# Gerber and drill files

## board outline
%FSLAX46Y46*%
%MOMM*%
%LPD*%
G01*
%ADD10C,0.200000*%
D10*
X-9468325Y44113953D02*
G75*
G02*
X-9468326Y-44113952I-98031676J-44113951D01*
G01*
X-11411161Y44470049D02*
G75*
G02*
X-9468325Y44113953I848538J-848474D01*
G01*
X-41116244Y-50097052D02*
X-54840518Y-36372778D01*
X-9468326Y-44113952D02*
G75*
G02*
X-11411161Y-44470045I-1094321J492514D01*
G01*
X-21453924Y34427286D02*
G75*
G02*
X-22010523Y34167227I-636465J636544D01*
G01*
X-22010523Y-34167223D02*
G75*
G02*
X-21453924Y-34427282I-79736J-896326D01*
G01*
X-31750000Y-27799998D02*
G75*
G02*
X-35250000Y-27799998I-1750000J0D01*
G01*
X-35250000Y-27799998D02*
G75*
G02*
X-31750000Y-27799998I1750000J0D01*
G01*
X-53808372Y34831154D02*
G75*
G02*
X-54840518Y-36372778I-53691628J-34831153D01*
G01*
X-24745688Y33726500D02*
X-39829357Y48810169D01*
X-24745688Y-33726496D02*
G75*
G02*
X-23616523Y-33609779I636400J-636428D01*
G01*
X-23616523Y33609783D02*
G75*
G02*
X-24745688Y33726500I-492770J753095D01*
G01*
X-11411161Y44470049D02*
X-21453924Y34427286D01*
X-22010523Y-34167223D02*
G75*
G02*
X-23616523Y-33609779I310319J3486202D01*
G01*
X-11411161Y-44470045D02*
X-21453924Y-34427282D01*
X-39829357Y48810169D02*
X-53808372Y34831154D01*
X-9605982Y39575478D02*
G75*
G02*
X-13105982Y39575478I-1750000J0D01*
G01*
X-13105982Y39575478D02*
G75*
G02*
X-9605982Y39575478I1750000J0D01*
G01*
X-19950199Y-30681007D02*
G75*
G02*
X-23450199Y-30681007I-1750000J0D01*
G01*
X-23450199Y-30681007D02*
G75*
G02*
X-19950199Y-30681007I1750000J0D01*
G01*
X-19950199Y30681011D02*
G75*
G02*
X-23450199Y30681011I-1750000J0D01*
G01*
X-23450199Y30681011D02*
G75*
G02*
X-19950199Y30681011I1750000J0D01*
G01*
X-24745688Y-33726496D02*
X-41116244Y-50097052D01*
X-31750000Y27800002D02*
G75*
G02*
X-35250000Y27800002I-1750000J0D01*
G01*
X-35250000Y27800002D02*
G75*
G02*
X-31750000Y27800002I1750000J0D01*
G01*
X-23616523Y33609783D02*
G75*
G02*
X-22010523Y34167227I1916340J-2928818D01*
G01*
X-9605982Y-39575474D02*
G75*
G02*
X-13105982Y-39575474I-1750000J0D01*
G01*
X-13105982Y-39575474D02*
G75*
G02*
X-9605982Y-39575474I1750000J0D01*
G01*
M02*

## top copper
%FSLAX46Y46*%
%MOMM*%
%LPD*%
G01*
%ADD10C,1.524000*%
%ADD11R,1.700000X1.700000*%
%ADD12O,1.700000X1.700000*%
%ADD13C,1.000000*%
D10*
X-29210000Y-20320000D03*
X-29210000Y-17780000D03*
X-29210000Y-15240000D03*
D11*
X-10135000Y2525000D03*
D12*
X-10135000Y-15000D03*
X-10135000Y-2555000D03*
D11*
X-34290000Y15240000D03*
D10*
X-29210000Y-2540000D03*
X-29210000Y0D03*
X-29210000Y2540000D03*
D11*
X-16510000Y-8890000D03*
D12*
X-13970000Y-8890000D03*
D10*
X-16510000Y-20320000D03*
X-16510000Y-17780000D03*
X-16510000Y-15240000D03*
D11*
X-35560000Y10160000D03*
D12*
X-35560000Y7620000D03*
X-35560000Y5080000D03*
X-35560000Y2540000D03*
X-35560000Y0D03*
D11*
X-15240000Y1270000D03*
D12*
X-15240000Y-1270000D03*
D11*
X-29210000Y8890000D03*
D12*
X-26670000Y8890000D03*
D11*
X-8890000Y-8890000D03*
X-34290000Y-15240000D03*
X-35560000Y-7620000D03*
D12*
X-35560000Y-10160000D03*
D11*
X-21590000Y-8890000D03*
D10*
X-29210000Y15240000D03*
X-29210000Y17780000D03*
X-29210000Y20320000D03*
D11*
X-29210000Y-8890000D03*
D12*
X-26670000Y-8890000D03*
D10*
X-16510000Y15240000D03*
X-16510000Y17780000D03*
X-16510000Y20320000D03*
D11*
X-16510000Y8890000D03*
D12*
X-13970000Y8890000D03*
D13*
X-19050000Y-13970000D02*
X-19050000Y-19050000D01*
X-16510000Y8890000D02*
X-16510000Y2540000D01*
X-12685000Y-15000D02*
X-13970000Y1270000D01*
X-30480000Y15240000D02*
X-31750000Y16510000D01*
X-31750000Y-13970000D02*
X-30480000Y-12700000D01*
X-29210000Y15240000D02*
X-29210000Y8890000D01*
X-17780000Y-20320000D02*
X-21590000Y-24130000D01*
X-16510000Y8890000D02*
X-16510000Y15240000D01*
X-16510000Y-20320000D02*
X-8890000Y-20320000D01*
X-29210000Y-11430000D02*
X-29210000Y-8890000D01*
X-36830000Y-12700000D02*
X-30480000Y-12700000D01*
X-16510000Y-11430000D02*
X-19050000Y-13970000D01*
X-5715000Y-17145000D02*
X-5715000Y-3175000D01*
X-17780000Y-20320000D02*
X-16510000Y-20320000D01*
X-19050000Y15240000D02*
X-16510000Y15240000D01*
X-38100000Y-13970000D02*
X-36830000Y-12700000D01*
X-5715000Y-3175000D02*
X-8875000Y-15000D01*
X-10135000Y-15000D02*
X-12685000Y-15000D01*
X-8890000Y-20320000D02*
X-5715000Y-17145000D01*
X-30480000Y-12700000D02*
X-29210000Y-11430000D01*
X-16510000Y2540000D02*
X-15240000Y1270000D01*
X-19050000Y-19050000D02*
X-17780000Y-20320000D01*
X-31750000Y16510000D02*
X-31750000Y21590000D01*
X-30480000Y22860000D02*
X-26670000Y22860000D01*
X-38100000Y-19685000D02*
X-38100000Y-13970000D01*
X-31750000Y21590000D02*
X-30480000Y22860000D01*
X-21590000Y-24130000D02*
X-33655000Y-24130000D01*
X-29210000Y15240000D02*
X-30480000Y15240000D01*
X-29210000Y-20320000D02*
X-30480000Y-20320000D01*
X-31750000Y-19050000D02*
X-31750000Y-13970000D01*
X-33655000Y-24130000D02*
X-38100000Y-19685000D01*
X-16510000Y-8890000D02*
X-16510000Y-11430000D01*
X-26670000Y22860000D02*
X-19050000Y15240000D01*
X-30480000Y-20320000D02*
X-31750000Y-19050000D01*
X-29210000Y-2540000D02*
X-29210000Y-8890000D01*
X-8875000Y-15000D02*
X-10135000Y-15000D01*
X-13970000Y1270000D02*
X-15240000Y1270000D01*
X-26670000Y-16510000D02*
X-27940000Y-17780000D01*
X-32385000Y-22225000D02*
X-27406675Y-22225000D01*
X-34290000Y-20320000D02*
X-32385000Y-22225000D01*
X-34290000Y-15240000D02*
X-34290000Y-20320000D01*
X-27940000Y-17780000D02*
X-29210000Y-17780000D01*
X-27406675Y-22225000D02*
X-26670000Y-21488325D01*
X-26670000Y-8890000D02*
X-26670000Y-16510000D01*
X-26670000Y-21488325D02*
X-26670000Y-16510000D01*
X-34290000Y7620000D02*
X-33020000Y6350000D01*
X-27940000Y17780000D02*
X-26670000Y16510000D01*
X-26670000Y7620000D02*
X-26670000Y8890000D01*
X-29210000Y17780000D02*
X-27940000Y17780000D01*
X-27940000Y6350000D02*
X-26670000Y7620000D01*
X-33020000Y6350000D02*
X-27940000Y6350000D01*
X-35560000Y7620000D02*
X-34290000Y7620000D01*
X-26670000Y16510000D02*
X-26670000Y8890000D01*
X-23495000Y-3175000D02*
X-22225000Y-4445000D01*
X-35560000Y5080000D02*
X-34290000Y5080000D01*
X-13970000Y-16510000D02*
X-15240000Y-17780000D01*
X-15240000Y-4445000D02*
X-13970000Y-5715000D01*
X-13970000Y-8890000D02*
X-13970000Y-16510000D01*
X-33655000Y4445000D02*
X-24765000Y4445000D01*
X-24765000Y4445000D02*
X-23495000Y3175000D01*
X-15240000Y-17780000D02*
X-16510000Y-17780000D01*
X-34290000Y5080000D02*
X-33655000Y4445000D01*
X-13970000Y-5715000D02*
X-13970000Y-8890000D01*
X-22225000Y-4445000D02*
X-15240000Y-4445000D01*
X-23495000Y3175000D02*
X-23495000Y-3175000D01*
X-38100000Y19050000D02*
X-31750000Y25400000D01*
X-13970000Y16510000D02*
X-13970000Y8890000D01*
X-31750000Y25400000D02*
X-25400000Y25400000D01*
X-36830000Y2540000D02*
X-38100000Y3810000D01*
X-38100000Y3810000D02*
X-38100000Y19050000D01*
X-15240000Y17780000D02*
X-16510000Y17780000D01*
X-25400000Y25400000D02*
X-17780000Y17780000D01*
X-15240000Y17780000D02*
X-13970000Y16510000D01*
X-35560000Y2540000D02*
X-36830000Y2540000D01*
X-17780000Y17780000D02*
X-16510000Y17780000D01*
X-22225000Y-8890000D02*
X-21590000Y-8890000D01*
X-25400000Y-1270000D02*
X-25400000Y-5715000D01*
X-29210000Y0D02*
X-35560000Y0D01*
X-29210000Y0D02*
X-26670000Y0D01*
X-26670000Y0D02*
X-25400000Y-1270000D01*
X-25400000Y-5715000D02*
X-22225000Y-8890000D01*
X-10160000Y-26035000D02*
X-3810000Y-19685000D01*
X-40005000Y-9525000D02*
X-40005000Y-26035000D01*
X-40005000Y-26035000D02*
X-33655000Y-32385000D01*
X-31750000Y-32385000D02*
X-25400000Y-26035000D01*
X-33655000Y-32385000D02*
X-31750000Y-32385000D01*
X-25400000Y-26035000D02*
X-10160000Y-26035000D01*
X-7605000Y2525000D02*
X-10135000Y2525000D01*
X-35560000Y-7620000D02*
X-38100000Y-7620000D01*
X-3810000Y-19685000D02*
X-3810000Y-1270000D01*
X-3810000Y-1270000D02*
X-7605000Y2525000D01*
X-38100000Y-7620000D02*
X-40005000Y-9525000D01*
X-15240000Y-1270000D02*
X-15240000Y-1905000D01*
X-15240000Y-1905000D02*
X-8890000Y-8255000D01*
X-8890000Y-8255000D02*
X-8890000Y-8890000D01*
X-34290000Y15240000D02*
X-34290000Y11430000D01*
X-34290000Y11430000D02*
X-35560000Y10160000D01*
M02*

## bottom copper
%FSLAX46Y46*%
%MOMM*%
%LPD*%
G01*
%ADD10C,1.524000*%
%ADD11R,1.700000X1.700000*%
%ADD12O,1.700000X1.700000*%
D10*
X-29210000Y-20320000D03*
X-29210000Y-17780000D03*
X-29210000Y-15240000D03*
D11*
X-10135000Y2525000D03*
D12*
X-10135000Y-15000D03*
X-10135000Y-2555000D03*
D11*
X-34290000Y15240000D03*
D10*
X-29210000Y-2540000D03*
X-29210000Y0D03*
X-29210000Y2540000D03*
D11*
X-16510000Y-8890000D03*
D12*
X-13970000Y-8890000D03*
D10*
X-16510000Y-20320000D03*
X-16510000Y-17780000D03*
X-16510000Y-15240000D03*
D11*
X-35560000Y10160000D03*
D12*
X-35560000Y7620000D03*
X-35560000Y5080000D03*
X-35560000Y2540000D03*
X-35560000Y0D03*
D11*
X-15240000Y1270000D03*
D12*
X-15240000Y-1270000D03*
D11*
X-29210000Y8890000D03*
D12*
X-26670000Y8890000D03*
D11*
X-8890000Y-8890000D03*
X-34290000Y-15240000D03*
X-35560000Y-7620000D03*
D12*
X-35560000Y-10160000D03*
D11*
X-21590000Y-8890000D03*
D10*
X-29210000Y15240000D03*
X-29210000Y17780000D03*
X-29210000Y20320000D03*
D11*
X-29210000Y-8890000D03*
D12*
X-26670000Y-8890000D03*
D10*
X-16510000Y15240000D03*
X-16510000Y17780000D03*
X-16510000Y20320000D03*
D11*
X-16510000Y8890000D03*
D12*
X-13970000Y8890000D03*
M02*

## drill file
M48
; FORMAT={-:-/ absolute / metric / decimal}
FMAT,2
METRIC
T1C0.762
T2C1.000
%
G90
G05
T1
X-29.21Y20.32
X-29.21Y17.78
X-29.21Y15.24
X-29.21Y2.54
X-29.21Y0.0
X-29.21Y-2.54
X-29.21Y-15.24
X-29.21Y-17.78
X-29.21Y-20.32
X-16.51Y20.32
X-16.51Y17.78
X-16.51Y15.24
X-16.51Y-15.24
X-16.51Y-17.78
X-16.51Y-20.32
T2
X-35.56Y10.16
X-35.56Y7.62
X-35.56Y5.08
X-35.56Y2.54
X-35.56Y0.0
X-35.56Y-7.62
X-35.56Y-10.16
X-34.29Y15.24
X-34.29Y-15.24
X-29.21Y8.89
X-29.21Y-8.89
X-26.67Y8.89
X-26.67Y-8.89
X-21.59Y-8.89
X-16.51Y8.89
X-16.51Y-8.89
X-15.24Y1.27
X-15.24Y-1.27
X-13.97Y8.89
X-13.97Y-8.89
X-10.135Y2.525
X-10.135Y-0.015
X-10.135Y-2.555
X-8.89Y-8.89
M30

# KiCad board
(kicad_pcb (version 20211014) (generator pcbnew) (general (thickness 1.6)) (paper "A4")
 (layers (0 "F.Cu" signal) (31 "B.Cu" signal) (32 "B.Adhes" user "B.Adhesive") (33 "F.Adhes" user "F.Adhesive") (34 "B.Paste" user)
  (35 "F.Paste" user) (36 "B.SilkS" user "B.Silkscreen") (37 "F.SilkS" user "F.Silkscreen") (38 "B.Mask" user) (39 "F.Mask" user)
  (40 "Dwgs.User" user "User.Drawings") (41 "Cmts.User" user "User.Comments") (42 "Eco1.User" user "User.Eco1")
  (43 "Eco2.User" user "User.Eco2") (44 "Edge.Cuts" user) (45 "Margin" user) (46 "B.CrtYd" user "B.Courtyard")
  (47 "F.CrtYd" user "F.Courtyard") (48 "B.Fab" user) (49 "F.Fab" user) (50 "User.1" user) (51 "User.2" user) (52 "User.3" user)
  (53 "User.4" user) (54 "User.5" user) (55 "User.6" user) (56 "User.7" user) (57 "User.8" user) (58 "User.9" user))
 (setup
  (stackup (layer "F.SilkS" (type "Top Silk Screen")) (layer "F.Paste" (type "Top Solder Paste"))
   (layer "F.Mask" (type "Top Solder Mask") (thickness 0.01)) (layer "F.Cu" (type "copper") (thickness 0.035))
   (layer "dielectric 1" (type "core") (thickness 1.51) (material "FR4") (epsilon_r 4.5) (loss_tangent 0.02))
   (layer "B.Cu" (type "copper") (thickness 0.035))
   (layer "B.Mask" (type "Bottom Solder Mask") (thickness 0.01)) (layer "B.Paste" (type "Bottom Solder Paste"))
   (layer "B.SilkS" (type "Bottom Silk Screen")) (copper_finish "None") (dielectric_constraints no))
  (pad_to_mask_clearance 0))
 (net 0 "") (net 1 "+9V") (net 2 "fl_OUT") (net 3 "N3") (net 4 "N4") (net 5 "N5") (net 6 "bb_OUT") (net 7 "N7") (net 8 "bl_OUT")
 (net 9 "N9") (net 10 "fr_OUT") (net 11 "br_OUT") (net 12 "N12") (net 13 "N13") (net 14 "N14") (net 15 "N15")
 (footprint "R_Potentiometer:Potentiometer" (layer "F.Cu") (at -31.75 17.78 90)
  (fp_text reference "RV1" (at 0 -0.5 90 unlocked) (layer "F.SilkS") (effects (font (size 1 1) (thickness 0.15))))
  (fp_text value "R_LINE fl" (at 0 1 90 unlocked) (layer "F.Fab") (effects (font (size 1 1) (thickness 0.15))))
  (pad "1" thru_hole circle (at -2.54 2.54 90) (size 1.524 1.524) (drill 0.762) (layers *.Cu *.Mask) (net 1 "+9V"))
  (pad "2" thru_hole circle (at 0 2.54 90) (size 1.524 1.524) (drill 0.762) (layers *.Cu *.Mask) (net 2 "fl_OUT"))
  (pad "3" thru_hole circle (at 2.54 2.54 90) (size 1.524 1.524) (drill 0.762) (layers *.Cu *.Mask) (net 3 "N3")))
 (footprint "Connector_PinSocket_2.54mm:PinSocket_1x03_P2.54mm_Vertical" (layer "F.Cu") (at -10.135 -2.525)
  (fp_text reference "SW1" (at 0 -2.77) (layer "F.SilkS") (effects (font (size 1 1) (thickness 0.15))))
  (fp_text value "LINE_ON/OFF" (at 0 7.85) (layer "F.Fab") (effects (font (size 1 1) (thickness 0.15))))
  (pad "1" thru_hole rect (at 0 0) (size 1.7 1.7) (drill 1) (layers *.Cu *.Mask) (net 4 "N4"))
  (pad "2" thru_hole oval (at 0 2.54) (size 1.7 1.7) (drill 1) (layers *.Cu *.Mask) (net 1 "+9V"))
  (pad "3" thru_hole oval (at 0 5.08) (size 1.7 1.7) (drill 1) (layers *.Cu *.Mask)))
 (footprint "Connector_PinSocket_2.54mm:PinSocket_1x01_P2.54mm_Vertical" (layer "F.Cu") (at -34.29 -15.24)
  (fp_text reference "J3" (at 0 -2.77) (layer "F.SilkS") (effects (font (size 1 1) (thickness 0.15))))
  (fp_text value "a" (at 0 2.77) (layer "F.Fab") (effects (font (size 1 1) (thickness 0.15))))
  (pad "1" thru_hole rect (at 0 0) (size 1.7 1.7) (drill 1) (layers *.Cu *.Mask) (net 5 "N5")))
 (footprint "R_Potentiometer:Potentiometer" (layer "F.Cu") (at -31.75 0 90)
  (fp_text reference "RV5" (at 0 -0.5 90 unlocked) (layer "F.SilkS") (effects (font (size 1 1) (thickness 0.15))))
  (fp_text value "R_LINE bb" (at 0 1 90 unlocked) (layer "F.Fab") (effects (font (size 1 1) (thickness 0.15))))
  (pad "1" thru_hole circle (at -2.54 2.54 90) (size 1.524 1.524) (drill 0.762) (layers *.Cu *.Mask) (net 1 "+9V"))
  (pad "2" thru_hole circle (at 0 2.54 90) (size 1.524 1.524) (drill 0.762) (layers *.Cu *.Mask) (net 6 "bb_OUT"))
  (pad "3" thru_hole circle (at 2.54 2.54 90) (size 1.524 1.524) (drill 0.762) (layers *.Cu *.Mask) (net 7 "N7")))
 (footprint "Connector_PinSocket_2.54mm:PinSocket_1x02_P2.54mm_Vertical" (layer "F.Cu") (at -16.51 8.89 90)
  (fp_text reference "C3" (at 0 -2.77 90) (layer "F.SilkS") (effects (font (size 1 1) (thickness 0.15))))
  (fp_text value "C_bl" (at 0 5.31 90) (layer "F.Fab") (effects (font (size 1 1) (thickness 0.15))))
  (pad "1" thru_hole rect (at 0 0 90) (size 1.7 1.7) (drill 1) (layers *.Cu *.Mask) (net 1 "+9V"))
  (pad "2" thru_hole oval (at 0 2.54 90) (size 1.7 1.7) (drill 1) (layers *.Cu *.Mask) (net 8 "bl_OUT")))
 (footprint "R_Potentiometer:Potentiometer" (layer "F.Cu") (at -19.05 17.78 90)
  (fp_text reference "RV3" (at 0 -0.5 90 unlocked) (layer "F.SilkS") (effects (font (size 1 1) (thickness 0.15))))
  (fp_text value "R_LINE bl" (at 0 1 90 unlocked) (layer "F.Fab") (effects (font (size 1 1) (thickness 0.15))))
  (pad "1" thru_hole circle (at -2.54 2.54 90) (size 1.524 1.524) (drill 0.762) (layers *.Cu *.Mask) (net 1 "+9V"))
  (pad "2" thru_hole circle (at 0 2.54 90) (size 1.524 1.524) (drill 0.762) (layers *.Cu *.Mask) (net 8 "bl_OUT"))
  (pad "3" thru_hole circle (at 2.54 2.54 90) (size 1.524 1.524) (drill 0.762) (layers *.Cu *.Mask) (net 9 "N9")))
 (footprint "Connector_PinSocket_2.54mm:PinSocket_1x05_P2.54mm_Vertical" (layer "F.Cu") (at -35.56 -10.16)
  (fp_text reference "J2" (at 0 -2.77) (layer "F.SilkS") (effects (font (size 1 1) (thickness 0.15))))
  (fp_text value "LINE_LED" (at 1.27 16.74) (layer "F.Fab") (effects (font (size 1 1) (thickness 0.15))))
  (pad "1" thru_hole rect (at 0 0) (size 1.7 1.7) (drill 1) (layers *.Cu *.Mask) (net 5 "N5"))
  (pad "2" thru_hole oval (at 0 2.54) (size 1.7 1.7) (drill 1) (layers *.Cu *.Mask) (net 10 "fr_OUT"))
  (pad "3" thru_hole oval (at 0 5.08) (size 1.7 1.7) (drill 1) (layers *.Cu *.Mask) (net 8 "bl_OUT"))
  (pad "4" thru_hole oval (at 0 7.62) (size 1.7 1.7) (drill 1) (layers *.Cu *.Mask) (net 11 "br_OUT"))
  (pad "5" thru_hole oval (at 0 10.16) (size 1.7 1.7) (drill 1) (layers *.Cu *.Mask) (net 6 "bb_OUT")))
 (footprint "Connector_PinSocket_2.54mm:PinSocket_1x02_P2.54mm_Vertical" (layer "F.Cu") (at -15.24 -1.27)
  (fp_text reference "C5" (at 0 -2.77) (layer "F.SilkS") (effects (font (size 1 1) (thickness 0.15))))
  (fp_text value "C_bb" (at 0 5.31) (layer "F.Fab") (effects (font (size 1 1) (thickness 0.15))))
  (pad "1" thru_hole rect (at 0 0) (size 1.7 1.7) (drill 1) (layers *.Cu *.Mask) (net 1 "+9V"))
  (pad "2" thru_hole oval (at 0 2.54) (size 1.7 1.7) (drill 1) (layers *.Cu *.Mask) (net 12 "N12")))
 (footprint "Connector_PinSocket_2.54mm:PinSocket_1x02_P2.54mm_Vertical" (layer "F.Cu") (at -29.21 -8.89 90)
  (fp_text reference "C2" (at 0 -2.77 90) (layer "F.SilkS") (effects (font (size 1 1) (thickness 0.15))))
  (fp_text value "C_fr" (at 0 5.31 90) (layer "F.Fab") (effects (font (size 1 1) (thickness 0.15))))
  (pad "1" thru_hole rect (at 0 0 90) (size 1.7 1.7) (drill 1) (layers *.Cu *.Mask) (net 1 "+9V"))
  (pad "2" thru_hole oval (at 0 2.54 90) (size 1.7 1.7) (drill 1) (layers *.Cu *.Mask) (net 10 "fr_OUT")))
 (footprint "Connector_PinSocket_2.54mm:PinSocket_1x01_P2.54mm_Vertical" (layer "F.Cu") (at -8.89 8.89)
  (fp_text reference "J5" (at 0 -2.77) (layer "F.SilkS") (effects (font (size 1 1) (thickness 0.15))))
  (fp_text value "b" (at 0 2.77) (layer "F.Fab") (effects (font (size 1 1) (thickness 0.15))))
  (pad "1" thru_hole rect (at 0 0) (size 1.7 1.7) (drill 1) (layers *.Cu *.Mask) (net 12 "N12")))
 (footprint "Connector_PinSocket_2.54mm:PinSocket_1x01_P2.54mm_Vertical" (layer "F.Cu") (at -34.29 15.24)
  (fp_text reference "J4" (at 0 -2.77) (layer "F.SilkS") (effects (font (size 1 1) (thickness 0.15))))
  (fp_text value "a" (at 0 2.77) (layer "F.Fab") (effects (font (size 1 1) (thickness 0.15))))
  (pad "1" thru_hole rect (at 0 0) (size 1.7 1.7) (drill 1) (layers *.Cu *.Mask) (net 2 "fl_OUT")))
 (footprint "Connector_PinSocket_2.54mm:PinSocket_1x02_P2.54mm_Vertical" (layer "F.Cu") (at -35.56 7.62)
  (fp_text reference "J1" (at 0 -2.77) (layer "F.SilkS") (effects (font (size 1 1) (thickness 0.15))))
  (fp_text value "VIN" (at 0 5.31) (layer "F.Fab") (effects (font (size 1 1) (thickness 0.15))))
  (pad "1" thru_hole rect (at 0 0) (size 1.7 1.7) (drill 1) (layers *.Cu *.Mask) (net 4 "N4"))
  (pad "2" thru_hole oval (at 0 2.54) (size 1.7 1.7) (drill 1) (layers *.Cu *.Mask) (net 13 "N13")))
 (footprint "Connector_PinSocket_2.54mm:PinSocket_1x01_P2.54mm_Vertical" (layer "F.Cu") (at -21.59 8.89)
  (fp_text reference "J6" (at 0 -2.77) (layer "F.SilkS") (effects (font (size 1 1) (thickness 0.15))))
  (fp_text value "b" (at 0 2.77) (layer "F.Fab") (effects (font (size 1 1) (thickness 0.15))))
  (pad "1" thru_hole rect (at 0 0) (size 1.7 1.7) (drill 1) (layers *.Cu *.Mask) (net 6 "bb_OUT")))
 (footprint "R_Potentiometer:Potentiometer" (layer "F.Cu") (at -31.75 -17.78 90)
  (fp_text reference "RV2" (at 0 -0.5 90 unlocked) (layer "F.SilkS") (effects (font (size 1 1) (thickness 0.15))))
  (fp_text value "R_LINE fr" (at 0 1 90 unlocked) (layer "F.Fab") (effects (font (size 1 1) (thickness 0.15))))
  (pad "1" thru_hole circle (at -2.54 2.54 90) (size 1.524 1.524) (drill 0.762) (layers *.Cu *.Mask) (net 1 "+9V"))
  (pad "2" thru_hole circle (at 0 2.54 90) (size 1.524 1.524) (drill 0.762) (layers *.Cu *.Mask) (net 10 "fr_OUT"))
  (pad "3" thru_hole circle (at 2.54 2.54 90) (size 1.524 1.524) (drill 0.762) (layers *.Cu *.Mask) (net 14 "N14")))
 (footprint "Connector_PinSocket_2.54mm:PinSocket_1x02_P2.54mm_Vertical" (layer "F.Cu") (at -29.21 8.89 90)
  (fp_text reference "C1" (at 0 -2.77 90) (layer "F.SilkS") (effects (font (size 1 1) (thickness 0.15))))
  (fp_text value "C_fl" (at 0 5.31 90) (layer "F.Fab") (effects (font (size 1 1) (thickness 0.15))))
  (pad "1" thru_hole rect (at 0 0 90) (size 1.7 1.7) (drill 1) (layers *.Cu *.Mask) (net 1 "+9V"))
  (pad "2" thru_hole oval (at 0 2.54 90) (size 1.7 1.7) (drill 1) (layers *.Cu *.Mask) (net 2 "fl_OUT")))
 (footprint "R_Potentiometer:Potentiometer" (layer "F.Cu") (at -19.05 -17.78 90)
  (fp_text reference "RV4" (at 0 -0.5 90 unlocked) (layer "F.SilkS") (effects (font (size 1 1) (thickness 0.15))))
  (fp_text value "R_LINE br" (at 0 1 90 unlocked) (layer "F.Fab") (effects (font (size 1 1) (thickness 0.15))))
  (pad "1" thru_hole circle (at -2.54 2.54 90) (size 1.524 1.524) (drill 0.762) (layers *.Cu *.Mask) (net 1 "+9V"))
  (pad "2" thru_hole circle (at 0 2.54 90) (size 1.524 1.524) (drill 0.762) (layers *.Cu *.Mask) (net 11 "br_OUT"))
  (pad "3" thru_hole circle (at 2.54 2.54 90) (size 1.524 1.524) (drill 0.762) (layers *.Cu *.Mask) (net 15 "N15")))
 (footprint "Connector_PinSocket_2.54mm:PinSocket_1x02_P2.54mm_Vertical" (layer "F.Cu") (at -16.51 -8.89 90)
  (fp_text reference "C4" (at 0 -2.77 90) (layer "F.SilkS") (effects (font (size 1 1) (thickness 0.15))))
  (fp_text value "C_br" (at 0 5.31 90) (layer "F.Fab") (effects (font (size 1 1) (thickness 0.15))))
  (pad "1" thru_hole rect (at 0 0 90) (size 1.7 1.7) (drill 1) (layers *.Cu *.Mask) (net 1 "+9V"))
  (pad "2" thru_hole oval (at 0 2.54 90) (size 1.7 1.7) (drill 1) (layers *.Cu *.Mask) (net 11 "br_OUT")))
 (gr_arc (start -9.468325 -44.113953) (mid 0 0) (end -9.468326 44.113952) (layer "Edge.Cuts") (width 0.2))
 (gr_arc (start -11.411161 -44.470049) (mid -10.346273 -44.801879) (end -9.468325 -44.113953) (layer "Edge.Cuts") (width 0.2))
 (gr_line (start -41.116244 50.097052) (end -54.840518 36.372778) (layer "Edge.Cuts") (width 0.2))
 (gr_arc (start -9.468326 44.113952) (mid -10.346285 44.801818) (end -11.411161 44.470045) (layer "Edge.Cuts") (width 0.2))
 (gr_arc (start -21.453924 -34.427286) (mid -21.709349 -34.248303) (end -22.010523 -34.167227) (layer "Edge.Cuts") (width 0.2))
 (gr_arc (start -22.010523 34.167223) (mid -21.709342 34.248282) (end -21.453924 34.427282) (layer "Edge.Cuts") (width 0.2))
 (gr_circle (center -33.5 27.799998) (end -31.75 27.799998) (layer "Edge.Cuts") (width 0.2) (fill none))
 (gr_arc (start -53.808372 -34.831154) (mid -43.506722 0.927622) (end -54.840518 36.372778) (layer "Edge.Cuts") (width 0.2))
 (gr_line (start -24.745688 -33.7265) (end -39.829357 -48.810169) (layer "Edge.Cuts") (width 0.2))
 (gr_arc (start -24.745688 33.726496) (mid -24.201829 33.467669) (end -23.616523 33.609779) (layer "Edge.Cuts") (width 0.2))
 (gr_arc (start -23.616523 -33.609783) (mid -24.20183 -33.467662) (end -24.745688 -33.7265) (layer "Edge.Cuts") (width 0.2))
 (gr_line (start -11.411161 -44.470049) (end -21.453924 -34.427286) (layer "Edge.Cuts") (width 0.2))
 (gr_arc (start -22.010523 34.167223) (mid -22.847882 33.98749) (end -23.616523 33.609779) (layer "Edge.Cuts") (width 0.2))
 (gr_line (start -11.411161 44.470045) (end -21.453924 34.427282) (layer "Edge.Cuts") (width 0.2))
 (gr_line (start -39.829357 -48.810169) (end -53.808372 -34.831154) (layer "Edge.Cuts") (width 0.2))
 (gr_circle (center -11.355982 -39.575478) (end -9.605982 -39.575478) (layer "Edge.Cuts") (width 0.2) (fill none))
 (gr_circle (center -21.700199 30.681007) (end -19.950199 30.681007) (layer "Edge.Cuts") (width 0.2) (fill none))
 (gr_circle (center -21.700199 -30.681011) (end -19.950199 -30.681011) (layer "Edge.Cuts") (width 0.2) (fill none))
 (gr_line (start -24.745688 33.726496) (end -41.116244 50.097052) (layer "Edge.Cuts") (width 0.2))
 (gr_circle (center -33.5 -27.800002) (end -31.75 -27.800002) (layer "Edge.Cuts") (width 0.2) (fill none))
 (gr_arc (start -23.616523 -33.609783) (mid -22.847882 -33.987492) (end -22.010523 -34.167227) (layer "Edge.Cuts") (width 0.2))
 (gr_circle (center -11.355982 39.575474) (end -9.605982 39.575474) (layer "Edge.Cuts") (width 0.2) (fill none))
 (segment (start -19.05 13.97) (end -19.05 19.05) (width 1) (layer "F.Cu") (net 1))
 (segment (start -16.51 -8.89) (end -16.51 -2.54) (width 1) (layer "F.Cu") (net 1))
 (segment (start -12.685 0.015) (end -13.97 -1.27) (width 1) (layer "F.Cu") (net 1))
 (segment (start -30.48 -15.24) (end -31.75 -16.51) (width 1) (layer "F.Cu") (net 1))
 (segment (start -31.75 13.97) (end -30.48 12.7) (width 1) (layer "F.Cu") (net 1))
 (segment (start -29.21 -15.24) (end -29.21 -8.89) (width 1) (layer "F.Cu") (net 1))
 (segment (start -17.78 20.32) (end -21.59 24.13) (width 1) (layer "F.Cu") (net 1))
 (segment (start -16.51 -8.89) (end -16.51 -15.24) (width 1) (layer "F.Cu") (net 1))
 (segment (start -16.51 20.32) (end -8.89 20.32) (width 1) (layer "F.Cu") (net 1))
 (segment (start -29.21 11.43) (end -29.21 8.89) (width 1) (layer "F.Cu") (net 1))
 (segment (start -36.83 12.7) (end -30.48 12.7) (width 1) (layer "F.Cu") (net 1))
 (segment (start -16.51 11.43) (end -19.05 13.97) (width 1) (layer "F.Cu") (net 1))
 (segment (start -5.715 17.145) (end -5.715 3.175) (width 1) (layer "F.Cu") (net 1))
 (segment (start -17.78 20.32) (end -16.51 20.32) (width 1) (layer "F.Cu") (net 1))
 (segment (start -19.05 -15.24) (end -16.51 -15.24) (width 1) (layer "F.Cu") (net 1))
 (segment (start -38.1 13.97) (end -36.83 12.7) (width 1) (layer "F.Cu") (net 1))
 (segment (start -5.715 3.175) (end -8.875 0.015) (width 1) (layer "F.Cu") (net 1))
 (segment (start -10.135 0.015) (end -12.685 0.015) (width 1) (layer "F.Cu") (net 1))
 (segment (start -8.89 20.32) (end -5.715 17.145) (width 1) (layer "F.Cu") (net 1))
 (segment (start -30.48 12.7) (end -29.21 11.43) (width 1) (layer "F.Cu") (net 1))
 (segment (start -16.51 -2.54) (end -15.24 -1.27) (width 1) (layer "F.Cu") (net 1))
 (segment (start -19.05 19.05) (end -17.78 20.32) (width 1) (layer "F.Cu") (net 1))
 (segment (start -31.75 -16.51) (end -31.75 -21.59) (width 1) (layer "F.Cu") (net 1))
 (segment (start -30.48 -22.86) (end -26.67 -22.86) (width 1) (layer "F.Cu") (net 1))
 (segment (start -38.1 19.685) (end -38.1 13.97) (width 1) (layer "F.Cu") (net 1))
 (segment (start -31.75 -21.59) (end -30.48 -22.86) (width 1) (layer "F.Cu") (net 1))
 (segment (start -21.59 24.13) (end -33.655 24.13) (width 1) (layer "F.Cu") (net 1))
 (segment (start -29.21 -15.24) (end -30.48 -15.24) (width 1) (layer "F.Cu") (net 1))
 (segment (start -29.21 20.32) (end -30.48 20.32) (width 1) (layer "F.Cu") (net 1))
 (segment (start -31.75 19.05) (end -31.75 13.97) (width 1) (layer "F.Cu") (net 1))
 (segment (start -33.655 24.13) (end -38.1 19.685) (width 1) (layer "F.Cu") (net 1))
 (segment (start -16.51 8.89) (end -16.51 11.43) (width 1) (layer "F.Cu") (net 1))
 (segment (start -26.67 -22.86) (end -19.05 -15.24) (width 1) (layer "F.Cu") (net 1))
 (segment (start -30.48 20.32) (end -31.75 19.05) (width 1) (layer "F.Cu") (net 1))
 (segment (start -29.21 2.54) (end -29.21 8.89) (width 1) (layer "F.Cu") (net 1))
 (segment (start -8.875 0.015) (end -10.135 0.015) (width 1) (layer "F.Cu") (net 1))
 (segment (start -13.97 -1.27) (end -15.24 -1.27) (width 1) (layer "F.Cu") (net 1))
 (segment (start -26.67 16.51) (end -27.94 17.78) (width 1) (layer "F.Cu") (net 2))
 (segment (start -32.385 22.225) (end -27.406675 22.225) (width 1) (layer "F.Cu") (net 2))
 (segment (start -34.29 20.32) (end -32.385 22.225) (width 1) (layer "F.Cu") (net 2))
 (segment (start -34.29 15.24) (end -34.29 20.32) (width 1) (layer "F.Cu") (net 2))
 (segment (start -27.94 17.78) (end -29.21 17.78) (width 1) (layer "F.Cu") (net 2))
 (segment (start -27.406675 22.225) (end -26.67 21.488325) (width 1) (layer "F.Cu") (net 2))
 (segment (start -26.67 8.89) (end -26.67 16.51) (width 1) (layer "F.Cu") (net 2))
 (segment (start -26.67 21.488325) (end -26.67 16.51) (width 1) (layer "F.Cu") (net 2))
 (segment (start -34.29 -7.62) (end -33.02 -6.35) (width 1) (layer "F.Cu") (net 10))
 (segment (start -27.94 -17.78) (end -26.67 -16.51) (width 1) (layer "F.Cu") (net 10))
 (segment (start -26.67 -7.62) (end -26.67 -8.89) (width 1) (layer "F.Cu") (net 10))
 (segment (start -29.21 -17.78) (end -27.94 -17.78) (width 1) (layer "F.Cu") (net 10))
 (segment (start -27.94 -6.35) (end -26.67 -7.62) (width 1) (layer "F.Cu") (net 10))
 (segment (start -33.02 -6.35) (end -27.94 -6.35) (width 1) (layer "F.Cu") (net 10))
 (segment (start -35.56 -7.62) (end -34.29 -7.62) (width 1) (layer "F.Cu") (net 10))
 (segment (start -26.67 -16.51) (end -26.67 -8.89) (width 1) (layer "F.Cu") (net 10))
 (segment (start -23.495 3.175) (end -22.225 4.445) (width 1) (layer "F.Cu") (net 8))
 (segment (start -35.56 -5.08) (end -34.29 -5.08) (width 1) (layer "F.Cu") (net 8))
 (segment (start -13.97 16.51) (end -15.24 17.78) (width 1) (layer "F.Cu") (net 8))
 (segment (start -15.24 4.445) (end -13.97 5.715) (width 1) (layer "F.Cu") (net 8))
 (segment (start -13.97 8.89) (end -13.97 16.51) (width 1) (layer "F.Cu") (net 8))
 (segment (start -33.655 -4.445) (end -24.765 -4.445) (width 1) (layer "F.Cu") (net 8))
 (segment (start -24.765 -4.445) (end -23.495 -3.175) (width 1) (layer "F.Cu") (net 8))
 (segment (start -15.24 17.78) (end -16.51 17.78) (width 1) (layer "F.Cu") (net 8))
 (segment (start -34.29 -5.08) (end -33.655 -4.445) (width 1) (layer "F.Cu") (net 8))
 (segment (start -13.97 5.715) (end -13.97 8.89) (width 1) (layer "F.Cu") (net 8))
 (segment (start -22.225 4.445) (end -15.24 4.445) (width 1) (layer "F.Cu") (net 8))
 (segment (start -23.495 -3.175) (end -23.495 3.175) (width 1) (layer "F.Cu") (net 8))
 (segment (start -38.1 -19.05) (end -31.75 -25.4) (width 1) (layer "F.Cu") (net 11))
 (segment (start -13.97 -16.51) (end -13.97 -8.89) (width 1) (layer "F.Cu") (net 11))
 (segment (start -31.75 -25.4) (end -25.4 -25.4) (width 1) (layer "F.Cu") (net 11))
 (segment (start -36.83 -2.54) (end -38.1 -3.81) (width 1) (layer "F.Cu") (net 11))
 (segment (start -38.1 -3.81) (end -38.1 -19.05) (width 1) (layer "F.Cu") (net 11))
 (segment (start -15.24 -17.78) (end -16.51 -17.78) (width 1) (layer "F.Cu") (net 11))
 (segment (start -25.4 -25.4) (end -17.78 -17.78) (width 1) (layer "F.Cu") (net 11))
 (segment (start -15.24 -17.78) (end -13.97 -16.51) (width 1) (layer "F.Cu") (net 11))
 (segment (start -35.56 -2.54) (end -36.83 -2.54) (width 1) (layer "F.Cu") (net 11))
 (segment (start -17.78 -17.78) (end -16.51 -17.78) (width 1) (layer "F.Cu") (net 11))
 (segment (start -22.225 8.89) (end -21.59 8.89) (width 1) (layer "F.Cu") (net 6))
 (segment (start -25.4 1.27) (end -25.4 5.715) (width 1) (layer "F.Cu") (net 6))
 (segment (start -29.21 0) (end -35.56 0) (width 1) (layer "F.Cu") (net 6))
 (segment (start -29.21 0) (end -26.67 0) (width 1) (layer "F.Cu") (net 6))
 (segment (start -26.67 0) (end -25.4 1.27) (width 1) (layer "F.Cu") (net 6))
 (segment (start -25.4 5.715) (end -22.225 8.89) (width 1) (layer "F.Cu") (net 6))
 (segment (start -10.16 26.035) (end -3.81 19.685) (width 1) (layer "F.Cu") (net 4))
 (segment (start -40.005 9.525) (end -40.005 26.035) (width 1) (layer "F.Cu") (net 4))
 (segment (start -40.005 26.035) (end -33.655 32.385) (width 1) (layer "F.Cu") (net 4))
 (segment (start -31.75 32.385) (end -25.4 26.035) (width 1) (layer "F.Cu") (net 4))
 (segment (start -33.655 32.385) (end -31.75 32.385) (width 1) (layer "F.Cu") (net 4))
 (segment (start -25.4 26.035) (end -10.16 26.035) (width 1) (layer "F.Cu") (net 4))
 (segment (start -7.605 -2.525) (end -10.135 -2.525) (width 1) (layer "F.Cu") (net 4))
 (segment (start -35.56 7.62) (end -38.1 7.62) (width 1) (layer "F.Cu") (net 4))
 (segment (start -3.81 19.685) (end -3.81 1.27) (width 1) (layer "F.Cu") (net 4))
 (segment (start -3.81 1.27) (end -7.605 -2.525) (width 1) (layer "F.Cu") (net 4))
 (segment (start -38.1 7.62) (end -40.005 9.525) (width 1) (layer "F.Cu") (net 4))
 (segment (start -15.24 1.27) (end -15.24 1.905) (width 1) (layer "F.Cu") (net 12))
 (segment (start -15.24 1.905) (end -8.89 8.255) (width 1) (layer "F.Cu") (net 12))
 (segment (start -8.89 8.255) (end -8.89 8.89) (width 1) (layer "F.Cu") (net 12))
 (segment (start -34.29 -15.24) (end -34.29 -11.43) (width 1) (layer "F.Cu") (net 5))
 (segment (start -34.29 -11.43) (end -35.56 -10.16) (width 1) (layer "F.Cu") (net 5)))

